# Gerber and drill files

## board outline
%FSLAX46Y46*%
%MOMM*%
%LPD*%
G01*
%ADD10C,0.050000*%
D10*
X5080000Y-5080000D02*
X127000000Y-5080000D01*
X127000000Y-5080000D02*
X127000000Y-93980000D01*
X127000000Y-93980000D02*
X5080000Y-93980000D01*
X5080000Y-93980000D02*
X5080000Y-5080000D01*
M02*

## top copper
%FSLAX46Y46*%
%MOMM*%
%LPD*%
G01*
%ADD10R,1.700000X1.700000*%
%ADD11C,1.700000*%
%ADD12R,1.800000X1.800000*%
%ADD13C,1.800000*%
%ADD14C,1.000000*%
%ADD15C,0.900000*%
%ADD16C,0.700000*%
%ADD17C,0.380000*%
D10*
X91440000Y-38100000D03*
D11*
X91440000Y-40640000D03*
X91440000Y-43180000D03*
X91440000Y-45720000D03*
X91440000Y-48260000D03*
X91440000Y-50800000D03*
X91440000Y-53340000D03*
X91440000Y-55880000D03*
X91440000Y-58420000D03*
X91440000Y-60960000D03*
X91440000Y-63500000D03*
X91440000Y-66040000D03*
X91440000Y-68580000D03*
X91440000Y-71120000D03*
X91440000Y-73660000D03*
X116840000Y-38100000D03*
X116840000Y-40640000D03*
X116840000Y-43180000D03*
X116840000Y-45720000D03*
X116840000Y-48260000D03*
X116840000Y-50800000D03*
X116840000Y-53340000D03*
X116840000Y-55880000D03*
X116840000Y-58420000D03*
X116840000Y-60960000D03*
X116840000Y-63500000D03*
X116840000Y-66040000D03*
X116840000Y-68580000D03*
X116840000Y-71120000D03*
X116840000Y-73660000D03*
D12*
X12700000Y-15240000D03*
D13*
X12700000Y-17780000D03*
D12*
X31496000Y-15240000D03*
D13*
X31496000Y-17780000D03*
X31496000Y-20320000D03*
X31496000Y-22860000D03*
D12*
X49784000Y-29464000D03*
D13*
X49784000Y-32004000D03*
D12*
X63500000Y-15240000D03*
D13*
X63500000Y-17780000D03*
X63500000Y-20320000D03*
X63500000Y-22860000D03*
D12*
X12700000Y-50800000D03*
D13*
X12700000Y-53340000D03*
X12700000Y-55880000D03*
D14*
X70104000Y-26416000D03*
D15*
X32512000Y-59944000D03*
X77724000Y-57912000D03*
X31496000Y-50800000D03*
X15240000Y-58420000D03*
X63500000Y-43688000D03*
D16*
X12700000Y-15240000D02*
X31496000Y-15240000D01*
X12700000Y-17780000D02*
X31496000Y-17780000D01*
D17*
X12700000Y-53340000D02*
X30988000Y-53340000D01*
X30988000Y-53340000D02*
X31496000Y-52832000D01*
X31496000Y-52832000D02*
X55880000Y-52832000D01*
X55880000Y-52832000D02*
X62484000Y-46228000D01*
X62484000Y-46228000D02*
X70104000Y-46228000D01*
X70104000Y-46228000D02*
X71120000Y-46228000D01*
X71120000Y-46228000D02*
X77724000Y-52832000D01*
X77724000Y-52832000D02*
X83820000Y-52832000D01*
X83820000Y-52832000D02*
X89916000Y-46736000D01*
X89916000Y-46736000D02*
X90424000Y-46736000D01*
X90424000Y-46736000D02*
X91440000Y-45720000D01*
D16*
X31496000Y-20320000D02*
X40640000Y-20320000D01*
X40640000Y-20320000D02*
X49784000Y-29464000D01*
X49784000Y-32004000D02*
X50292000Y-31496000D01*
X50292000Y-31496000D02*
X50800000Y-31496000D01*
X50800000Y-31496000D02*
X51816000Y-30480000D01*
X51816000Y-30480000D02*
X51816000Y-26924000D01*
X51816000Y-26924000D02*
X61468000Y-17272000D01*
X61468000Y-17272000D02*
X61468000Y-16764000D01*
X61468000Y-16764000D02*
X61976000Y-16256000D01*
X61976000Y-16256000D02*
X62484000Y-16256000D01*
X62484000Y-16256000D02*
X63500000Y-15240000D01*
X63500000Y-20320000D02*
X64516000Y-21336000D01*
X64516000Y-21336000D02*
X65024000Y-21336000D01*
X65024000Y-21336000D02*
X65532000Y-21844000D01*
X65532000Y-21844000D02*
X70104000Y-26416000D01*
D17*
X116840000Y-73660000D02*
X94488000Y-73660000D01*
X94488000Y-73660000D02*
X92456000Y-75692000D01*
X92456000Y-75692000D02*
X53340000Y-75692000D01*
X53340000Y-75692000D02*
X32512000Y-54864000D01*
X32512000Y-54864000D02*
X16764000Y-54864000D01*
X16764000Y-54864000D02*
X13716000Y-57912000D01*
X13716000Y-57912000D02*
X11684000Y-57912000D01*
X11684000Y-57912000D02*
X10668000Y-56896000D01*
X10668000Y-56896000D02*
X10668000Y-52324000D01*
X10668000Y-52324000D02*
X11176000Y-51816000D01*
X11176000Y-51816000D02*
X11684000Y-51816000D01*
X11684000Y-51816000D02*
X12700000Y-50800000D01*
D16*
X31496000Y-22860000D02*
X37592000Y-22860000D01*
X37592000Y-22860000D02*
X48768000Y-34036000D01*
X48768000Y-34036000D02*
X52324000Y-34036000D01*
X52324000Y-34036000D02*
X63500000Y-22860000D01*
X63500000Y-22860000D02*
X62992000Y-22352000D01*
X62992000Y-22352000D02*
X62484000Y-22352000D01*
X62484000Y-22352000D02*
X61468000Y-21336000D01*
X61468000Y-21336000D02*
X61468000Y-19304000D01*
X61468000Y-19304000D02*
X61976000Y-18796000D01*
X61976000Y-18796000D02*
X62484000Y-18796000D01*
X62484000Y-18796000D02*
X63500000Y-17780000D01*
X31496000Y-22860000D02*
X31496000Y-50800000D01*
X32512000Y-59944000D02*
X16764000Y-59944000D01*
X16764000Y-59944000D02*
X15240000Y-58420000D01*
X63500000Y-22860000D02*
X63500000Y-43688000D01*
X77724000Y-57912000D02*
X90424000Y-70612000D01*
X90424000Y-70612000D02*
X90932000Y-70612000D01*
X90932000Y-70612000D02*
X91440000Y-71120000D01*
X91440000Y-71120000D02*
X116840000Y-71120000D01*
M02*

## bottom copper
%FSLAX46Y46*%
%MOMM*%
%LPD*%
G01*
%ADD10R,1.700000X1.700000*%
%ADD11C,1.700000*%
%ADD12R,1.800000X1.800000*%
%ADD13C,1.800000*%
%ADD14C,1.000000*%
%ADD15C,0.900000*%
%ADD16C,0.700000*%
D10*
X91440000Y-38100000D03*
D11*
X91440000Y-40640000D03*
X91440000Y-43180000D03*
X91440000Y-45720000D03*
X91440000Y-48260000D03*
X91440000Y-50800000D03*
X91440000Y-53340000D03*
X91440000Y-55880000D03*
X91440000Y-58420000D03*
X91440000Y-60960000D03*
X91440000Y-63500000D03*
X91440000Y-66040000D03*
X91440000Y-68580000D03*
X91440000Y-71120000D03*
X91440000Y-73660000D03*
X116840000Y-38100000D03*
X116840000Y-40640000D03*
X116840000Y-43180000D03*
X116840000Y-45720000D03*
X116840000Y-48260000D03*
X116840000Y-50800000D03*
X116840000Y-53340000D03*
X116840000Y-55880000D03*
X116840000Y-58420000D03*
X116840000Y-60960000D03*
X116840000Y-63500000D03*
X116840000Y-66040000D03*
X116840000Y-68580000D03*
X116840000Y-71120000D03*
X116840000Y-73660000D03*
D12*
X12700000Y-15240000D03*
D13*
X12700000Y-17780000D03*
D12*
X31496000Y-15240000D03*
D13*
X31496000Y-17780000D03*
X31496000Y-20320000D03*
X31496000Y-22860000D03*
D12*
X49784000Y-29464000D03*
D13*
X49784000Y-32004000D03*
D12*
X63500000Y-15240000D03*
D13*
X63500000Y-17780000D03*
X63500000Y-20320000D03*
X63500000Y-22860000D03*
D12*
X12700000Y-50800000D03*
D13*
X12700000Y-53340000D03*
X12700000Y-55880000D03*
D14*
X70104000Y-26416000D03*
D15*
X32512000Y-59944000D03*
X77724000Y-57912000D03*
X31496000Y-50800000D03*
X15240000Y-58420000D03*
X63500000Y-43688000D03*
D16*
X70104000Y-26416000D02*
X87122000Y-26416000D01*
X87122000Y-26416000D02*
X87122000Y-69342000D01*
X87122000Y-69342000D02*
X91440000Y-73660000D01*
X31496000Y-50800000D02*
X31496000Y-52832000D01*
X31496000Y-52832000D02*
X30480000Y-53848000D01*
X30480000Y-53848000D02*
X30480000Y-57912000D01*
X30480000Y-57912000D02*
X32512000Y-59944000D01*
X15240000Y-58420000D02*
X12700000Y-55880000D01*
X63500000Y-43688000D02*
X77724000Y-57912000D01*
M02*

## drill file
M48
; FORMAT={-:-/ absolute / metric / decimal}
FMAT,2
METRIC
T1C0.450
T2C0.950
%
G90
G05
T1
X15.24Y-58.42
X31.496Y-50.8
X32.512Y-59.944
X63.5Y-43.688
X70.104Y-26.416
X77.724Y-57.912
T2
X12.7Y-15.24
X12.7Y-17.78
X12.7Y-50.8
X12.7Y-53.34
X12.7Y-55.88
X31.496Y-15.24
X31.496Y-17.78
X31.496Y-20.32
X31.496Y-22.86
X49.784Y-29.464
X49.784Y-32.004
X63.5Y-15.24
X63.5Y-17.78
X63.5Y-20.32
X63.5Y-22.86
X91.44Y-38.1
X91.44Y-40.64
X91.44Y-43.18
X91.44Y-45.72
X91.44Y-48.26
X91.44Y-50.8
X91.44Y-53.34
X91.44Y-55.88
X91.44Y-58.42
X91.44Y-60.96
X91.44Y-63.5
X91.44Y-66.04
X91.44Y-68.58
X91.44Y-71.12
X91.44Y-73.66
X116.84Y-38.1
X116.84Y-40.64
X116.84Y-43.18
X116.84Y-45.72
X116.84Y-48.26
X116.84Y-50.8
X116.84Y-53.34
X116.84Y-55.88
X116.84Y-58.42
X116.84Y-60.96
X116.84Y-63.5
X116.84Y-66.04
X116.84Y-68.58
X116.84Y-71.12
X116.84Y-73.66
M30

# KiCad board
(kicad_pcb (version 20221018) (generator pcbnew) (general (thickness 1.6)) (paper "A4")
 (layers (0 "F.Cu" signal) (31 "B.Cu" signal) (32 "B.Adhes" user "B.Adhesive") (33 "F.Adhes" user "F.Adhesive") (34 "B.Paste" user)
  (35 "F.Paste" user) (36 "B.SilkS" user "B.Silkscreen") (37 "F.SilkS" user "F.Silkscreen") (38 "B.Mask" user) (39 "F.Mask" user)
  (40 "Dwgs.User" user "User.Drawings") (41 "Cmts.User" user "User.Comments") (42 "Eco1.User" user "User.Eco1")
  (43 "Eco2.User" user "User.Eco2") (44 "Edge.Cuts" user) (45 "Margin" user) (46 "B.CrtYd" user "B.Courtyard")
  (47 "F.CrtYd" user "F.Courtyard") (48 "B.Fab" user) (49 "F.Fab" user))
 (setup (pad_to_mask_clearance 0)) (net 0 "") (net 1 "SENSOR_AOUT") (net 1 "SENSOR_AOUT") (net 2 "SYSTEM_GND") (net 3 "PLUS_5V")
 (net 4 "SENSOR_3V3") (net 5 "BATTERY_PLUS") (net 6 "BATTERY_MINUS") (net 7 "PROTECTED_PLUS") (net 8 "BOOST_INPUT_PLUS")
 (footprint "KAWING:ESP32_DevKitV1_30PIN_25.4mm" (layer "F.Cu") (at 91.44 38.1)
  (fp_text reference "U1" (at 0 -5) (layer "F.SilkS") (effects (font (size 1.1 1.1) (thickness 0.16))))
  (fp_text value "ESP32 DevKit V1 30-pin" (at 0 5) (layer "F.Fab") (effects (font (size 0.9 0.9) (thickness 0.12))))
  (pad "1" thru_hole rect (at 0 0) (size 1.7 1.7) (drill 0.95) (layers "*.Cu" "*.Mask"))
  (pad "2" thru_hole circle (at 0 2.54) (size 1.7 1.7) (drill 0.95) (layers "*.Cu" "*.Mask"))
  (pad "3" thru_hole circle (at 0 5.08) (size 1.7 1.7) (drill 0.95) (layers "*.Cu" "*.Mask"))
  (pad "4" thru_hole circle (at 0 7.62) (size 1.7 1.7) (drill 0.95) (layers "*.Cu" "*.Mask") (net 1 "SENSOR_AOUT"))
  (pad "5" thru_hole circle (at 0 10.16) (size 1.7 1.7) (drill 0.95) (layers "*.Cu" "*.Mask"))
  (pad "6" thru_hole circle (at 0 12.7) (size 1.7 1.7) (drill 0.95) (layers "*.Cu" "*.Mask"))
  (pad "7" thru_hole circle (at 0 15.24) (size 1.7 1.7) (drill 0.95) (layers "*.Cu" "*.Mask"))
  (pad "8" thru_hole circle (at 0 17.78) (size 1.7 1.7) (drill 0.95) (layers "*.Cu" "*.Mask"))
  (pad "9" thru_hole circle (at 0 20.32) (size 1.7 1.7) (drill 0.95) (layers "*.Cu" "*.Mask"))
  (pad "10" thru_hole circle (at 0 22.86) (size 1.7 1.7) (drill 0.95) (layers "*.Cu" "*.Mask"))
  (pad "11" thru_hole circle (at 0 25.4) (size 1.7 1.7) (drill 0.95) (layers "*.Cu" "*.Mask"))
  (pad "12" thru_hole circle (at 0 27.94) (size 1.7 1.7) (drill 0.95) (layers "*.Cu" "*.Mask"))
  (pad "13" thru_hole circle (at 0 30.48) (size 1.7 1.7) (drill 0.95) (layers "*.Cu" "*.Mask"))
  (pad "14" thru_hole circle (at 0 33.02) (size 1.7 1.7) (drill 0.95) (layers "*.Cu" "*.Mask") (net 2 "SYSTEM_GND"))
  (pad "15" thru_hole circle (at 0 35.56) (size 1.7 1.7) (drill 0.95) (layers "*.Cu" "*.Mask") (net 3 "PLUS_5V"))
  (pad "16" thru_hole circle (at 25.4 0) (size 1.7 1.7) (drill 0.95) (layers "*.Cu" "*.Mask"))
  (pad "17" thru_hole circle (at 25.4 2.54) (size 1.7 1.7) (drill 0.95) (layers "*.Cu" "*.Mask"))
  (pad "18" thru_hole circle (at 25.4 5.08) (size 1.7 1.7) (drill 0.95) (layers "*.Cu" "*.Mask"))
  (pad "19" thru_hole circle (at 25.4 7.62) (size 1.7 1.7) (drill 0.95) (layers "*.Cu" "*.Mask"))
  (pad "20" thru_hole circle (at 25.4 10.16) (size 1.7 1.7) (drill 0.95) (layers "*.Cu" "*.Mask"))
  (pad "21" thru_hole circle (at 25.4 12.7) (size 1.7 1.7) (drill 0.95) (layers "*.Cu" "*.Mask"))
  (pad "22" thru_hole circle (at 25.4 15.24) (size 1.7 1.7) (drill 0.95) (layers "*.Cu" "*.Mask"))
  (pad "23" thru_hole circle (at 25.4 17.78) (size 1.7 1.7) (drill 0.95) (layers "*.Cu" "*.Mask"))
  (pad "24" thru_hole circle (at 25.4 20.32) (size 1.7 1.7) (drill 0.95) (layers "*.Cu" "*.Mask"))
  (pad "25" thru_hole circle (at 25.4 22.86) (size 1.7 1.7) (drill 0.95) (layers "*.Cu" "*.Mask"))
  (pad "26" thru_hole circle (at 25.4 25.4) (size 1.7 1.7) (drill 0.95) (layers "*.Cu" "*.Mask"))
  (pad "27" thru_hole circle (at 25.4 27.94) (size 1.7 1.7) (drill 0.95) (layers "*.Cu" "*.Mask"))
  (pad "28" thru_hole circle (at 25.4 30.48) (size 1.7 1.7) (drill 0.95) (layers "*.Cu" "*.Mask"))
  (pad "29" thru_hole circle (at 25.4 33.02) (size 1.7 1.7) (drill 0.95) (layers "*.Cu" "*.Mask") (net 2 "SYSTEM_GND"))
  (pad "30" thru_hole circle (at 25.4 35.56) (size 1.7 1.7) (drill 0.95) (layers "*.Cu" "*.Mask") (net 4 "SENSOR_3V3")))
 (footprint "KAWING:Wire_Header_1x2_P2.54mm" (layer "F.Cu") (at 12.7 15.24)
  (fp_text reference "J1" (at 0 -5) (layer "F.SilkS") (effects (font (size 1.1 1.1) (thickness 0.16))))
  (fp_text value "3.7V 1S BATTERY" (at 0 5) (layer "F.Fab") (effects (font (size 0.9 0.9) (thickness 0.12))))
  (pad "1" thru_hole rect (at 0 0) (size 1.8 1.8) (drill 0.95) (layers "*.Cu" "*.Mask") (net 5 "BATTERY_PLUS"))
  (pad "2" thru_hole circle (at 0 2.54) (size 1.8 1.8) (drill 0.95) (layers "*.Cu" "*.Mask") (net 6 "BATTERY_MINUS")))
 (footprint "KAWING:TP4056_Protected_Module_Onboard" (layer "F.Cu") (at 31.496 15.24)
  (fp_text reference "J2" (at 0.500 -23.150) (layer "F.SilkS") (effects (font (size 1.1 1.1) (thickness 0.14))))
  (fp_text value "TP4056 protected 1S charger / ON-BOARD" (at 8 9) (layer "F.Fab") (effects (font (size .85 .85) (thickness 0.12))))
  (pad "1" thru_hole rect (at 0.0 0.0) (size 1.8 1.8) (drill 0.95) (layers "*.Cu" "*.Mask") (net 5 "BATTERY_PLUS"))
  (pad "2" thru_hole circle (at 0.0 2.54) (size 1.8 1.8) (drill 0.95) (layers "*.Cu" "*.Mask") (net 6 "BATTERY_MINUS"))
  (pad "3" thru_hole circle (at 0.0 5.08) (size 1.8 1.8) (drill 0.95) (layers "*.Cu" "*.Mask") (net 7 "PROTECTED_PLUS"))
  (pad "4" thru_hole circle (at 0.0 7.62) (size 1.8 1.8) (drill 0.95) (layers "*.Cu" "*.Mask") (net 2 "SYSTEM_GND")))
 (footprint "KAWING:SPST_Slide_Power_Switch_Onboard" (layer "F.Cu") (at 49.784 29.464)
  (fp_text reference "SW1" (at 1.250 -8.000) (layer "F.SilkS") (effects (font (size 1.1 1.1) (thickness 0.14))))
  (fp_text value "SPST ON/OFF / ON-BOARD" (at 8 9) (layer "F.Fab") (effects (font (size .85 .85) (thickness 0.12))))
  (pad "1" thru_hole rect (at 0.0 0.0) (size 1.8 1.8) (drill 0.95) (layers "*.Cu" "*.Mask") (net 7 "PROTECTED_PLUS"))
  (pad "2" thru_hole circle (at 0.0 2.54) (size 1.8 1.8) (drill 0.95) (layers "*.Cu" "*.Mask") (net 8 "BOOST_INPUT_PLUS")))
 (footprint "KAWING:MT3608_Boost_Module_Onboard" (layer "F.Cu") (at 63.5 15.24)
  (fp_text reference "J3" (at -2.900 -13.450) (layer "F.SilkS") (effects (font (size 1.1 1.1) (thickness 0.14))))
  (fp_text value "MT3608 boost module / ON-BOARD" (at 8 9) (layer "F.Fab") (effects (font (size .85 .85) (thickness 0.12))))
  (pad "1" thru_hole rect (at 0.0 0.0) (size 1.8 1.8) (drill 0.95) (layers "*.Cu" "*.Mask") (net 8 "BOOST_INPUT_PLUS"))
  (pad "2" thru_hole circle (at 0.0 2.54) (size 1.8 1.8) (drill 0.95) (layers "*.Cu" "*.Mask") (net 2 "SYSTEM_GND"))
  (pad "3" thru_hole circle (at 0.0 5.08) (size 1.8 1.8) (drill 0.95) (layers "*.Cu" "*.Mask") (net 3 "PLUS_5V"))
  (pad "4" thru_hole circle (at 0.0 7.62) (size 1.8 1.8) (drill 0.95) (layers "*.Cu" "*.Mask") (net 2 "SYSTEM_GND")))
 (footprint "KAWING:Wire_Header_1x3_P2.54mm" (layer "F.Cu") (at 12.7 50.8)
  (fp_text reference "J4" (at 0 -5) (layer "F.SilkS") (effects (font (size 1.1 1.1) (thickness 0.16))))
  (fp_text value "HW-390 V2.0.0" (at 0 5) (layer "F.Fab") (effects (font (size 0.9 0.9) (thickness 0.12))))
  (pad "1" thru_hole rect (at 0 0) (size 1.8 1.8) (drill 0.95) (layers "*.Cu" "*.Mask") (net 4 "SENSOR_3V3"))
  (pad "2" thru_hole circle (at 0 2.54) (size 1.8 1.8) (drill 0.95) (layers "*.Cu" "*.Mask") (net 1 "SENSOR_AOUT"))
  (pad "3" thru_hole circle (at 0 5.08) (size 1.8 1.8) (drill 0.95) (layers "*.Cu" "*.Mask") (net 2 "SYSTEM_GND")))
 (gr_line (start 5.08 5.08) (end 127 5.08) (stroke (width 0.05) (type default)) (layer "Edge.Cuts"))
 (gr_line (start 127 5.08) (end 127 93.98) (stroke (width 0.05) (type default)) (layer "Edge.Cuts"))
 (gr_line (start 127 93.98) (end 5.08 93.98) (stroke (width 0.05) (type default)) (layer "Edge.Cuts"))
 (gr_line (start 5.08 93.98) (end 5.08 5.08) (stroke (width 0.05) (type default)) (layer "Edge.Cuts"))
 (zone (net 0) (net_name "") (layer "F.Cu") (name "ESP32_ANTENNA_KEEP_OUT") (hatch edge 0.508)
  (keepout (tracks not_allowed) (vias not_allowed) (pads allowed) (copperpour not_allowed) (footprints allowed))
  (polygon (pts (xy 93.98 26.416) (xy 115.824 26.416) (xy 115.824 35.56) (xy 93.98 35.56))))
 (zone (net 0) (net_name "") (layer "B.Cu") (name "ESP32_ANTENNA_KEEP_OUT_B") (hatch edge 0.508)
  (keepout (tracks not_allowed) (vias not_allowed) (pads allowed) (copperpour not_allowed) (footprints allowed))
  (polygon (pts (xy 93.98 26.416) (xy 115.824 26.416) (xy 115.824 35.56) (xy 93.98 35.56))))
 (segment (start 12.7 15.24) (end 31.496 15.24) (width 0.7) (layer "F.Cu") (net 5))
 (segment (start 12.7 17.78) (end 31.496 17.78) (width 0.7) (layer "F.Cu") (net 6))
 (segment (start 12.7 53.34) (end 30.988 53.34) (width 0.38) (layer "F.Cu") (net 1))
 (segment (start 30.988 53.34) (end 31.496 52.832) (width 0.38) (layer "F.Cu") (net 1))
 (segment (start 31.496 52.832) (end 55.88 52.832) (width 0.38) (layer "F.Cu") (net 1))
 (segment (start 55.88 52.832) (end 62.484 46.228) (width 0.38) (layer "F.Cu") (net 1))
 (segment (start 62.484 46.228) (end 70.104 46.228) (width 0.38) (layer "F.Cu") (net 1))
 (segment (start 70.104 46.228) (end 71.12 46.228) (width 0.38) (layer "F.Cu") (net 1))
 (segment (start 71.12 46.228) (end 77.724 52.832) (width 0.38) (layer "F.Cu") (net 1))
 (segment (start 77.724 52.832) (end 83.82 52.832) (width 0.38) (layer "F.Cu") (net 1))
 (segment (start 83.82 52.832) (end 89.916 46.736) (width 0.38) (layer "F.Cu") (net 1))
 (segment (start 89.916 46.736) (end 90.424 46.736) (width 0.38) (layer "F.Cu") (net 1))
 (segment (start 90.424 46.736) (end 91.44 45.72) (width 0.38) (layer "F.Cu") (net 1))
 (segment (start 31.496 20.32) (end 40.64 20.32) (width 0.7) (layer "F.Cu") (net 7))
 (segment (start 40.64 20.32) (end 49.784 29.464) (width 0.7) (layer "F.Cu") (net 7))
 (segment (start 49.784 32.004) (end 50.292 31.496) (width 0.7) (layer "F.Cu") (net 8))
 (segment (start 50.292 31.496) (end 50.8 31.496) (width 0.7) (layer "F.Cu") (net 8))
 (segment (start 50.8 31.496) (end 51.816 30.48) (width 0.7) (layer "F.Cu") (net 8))
 (segment (start 51.816 30.48) (end 51.816 26.924) (width 0.7) (layer "F.Cu") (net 8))
 (segment (start 51.816 26.924) (end 61.468 17.272) (width 0.7) (layer "F.Cu") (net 8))
 (segment (start 61.468 17.272) (end 61.468 16.764) (width 0.7) (layer "F.Cu") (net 8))
 (segment (start 61.468 16.764) (end 61.976 16.256) (width 0.7) (layer "F.Cu") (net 8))
 (segment (start 61.976 16.256) (end 62.484 16.256) (width 0.7) (layer "F.Cu") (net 8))
 (segment (start 62.484 16.256) (end 63.5 15.24) (width 0.7) (layer "F.Cu") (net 8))
 (segment (start 63.5 20.32) (end 64.516 21.336) (width 0.7) (layer "F.Cu") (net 3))
 (segment (start 64.516 21.336) (end 65.024 21.336) (width 0.7) (layer "F.Cu") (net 3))
 (segment (start 65.024 21.336) (end 65.532 21.844) (width 0.7) (layer "F.Cu") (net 3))
 (segment (start 65.532 21.844) (end 70.104 26.416) (width 0.7) (layer "F.Cu") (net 3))
 (segment (start 70.104 26.416) (end 87.122 26.416) (width 0.7) (layer "B.Cu") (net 3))
 (segment (start 87.122 26.416) (end 87.122 69.342) (width 0.7) (layer "B.Cu") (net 3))
 (segment (start 87.122 69.342) (end 91.44 73.66) (width 0.7) (layer "B.Cu") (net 3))
 (via (at 70.104 26.416) (size 1.0) (drill 0.45) (layers "F.Cu" "B.Cu") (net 3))
 (segment (start 116.84 73.66) (end 94.488 73.66) (width 0.38) (layer "F.Cu") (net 4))
 (segment (start 94.488 73.66) (end 92.456 75.692) (width 0.38) (layer "F.Cu") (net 4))
 (segment (start 92.456 75.692) (end 53.34 75.692) (width 0.38) (layer "F.Cu") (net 4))
 (segment (start 53.34 75.692) (end 32.512 54.864) (width 0.38) (layer "F.Cu") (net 4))
 (segment (start 32.512 54.864) (end 16.764 54.864) (width 0.38) (layer "F.Cu") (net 4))
 (segment (start 16.764 54.864) (end 13.716 57.912) (width 0.38) (layer "F.Cu") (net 4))
 (segment (start 13.716 57.912) (end 11.684 57.912) (width 0.38) (layer "F.Cu") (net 4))
 (segment (start 11.684 57.912) (end 10.668 56.896) (width 0.38) (layer "F.Cu") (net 4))
 (segment (start 10.668 56.896) (end 10.668 52.324) (width 0.38) (layer "F.Cu") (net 4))
 (segment (start 10.668 52.324) (end 11.176 51.816) (width 0.38) (layer "F.Cu") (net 4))
 (segment (start 11.176 51.816) (end 11.684 51.816) (width 0.38) (layer "F.Cu") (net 4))
 (segment (start 11.684 51.816) (end 12.7 50.8) (width 0.38) (layer "F.Cu") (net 4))
 (via (at 32.512 59.944) (size 0.9) (drill 0.45) (layers "F.Cu" "B.Cu") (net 2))
 (via (at 77.724 57.912) (size 0.9) (drill 0.45) (layers "F.Cu" "B.Cu") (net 2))
 (segment (start 31.496 22.86) (end 37.592 22.86) (width 0.7) (layer "F.Cu") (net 2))
 (segment (start 37.592 22.86) (end 48.768 34.036) (width 0.7) (layer "F.Cu") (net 2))
 (segment (start 48.768 34.036) (end 52.324 34.036) (width 0.7) (layer "F.Cu") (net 2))
 (segment (start 52.324 34.036) (end 63.5 22.86) (width 0.7) (layer "F.Cu") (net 2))
 (segment (start 63.5 22.86) (end 62.992 22.352) (width 0.7) (layer "F.Cu") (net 2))
 (segment (start 62.992 22.352) (end 62.484 22.352) (width 0.7) (layer "F.Cu") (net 2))
 (segment (start 62.484 22.352) (end 61.468 21.336) (width 0.7) (layer "F.Cu") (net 2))
 (segment (start 61.468 21.336) (end 61.468 19.304) (width 0.7) (layer "F.Cu") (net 2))
 (segment (start 61.468 19.304) (end 61.976 18.796) (width 0.7) (layer "F.Cu") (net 2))
 (segment (start 61.976 18.796) (end 62.484 18.796) (width 0.7) (layer "F.Cu") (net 2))
 (segment (start 62.484 18.796) (end 63.5 17.78) (width 0.7) (layer "F.Cu") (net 2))
 (segment (start 31.496 22.86) (end 31.496 50.8) (width 0.7) (layer "F.Cu") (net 2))
 (segment (start 31.496 50.8) (end 31.496 52.832) (width 0.7) (layer "B.Cu") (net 2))
 (segment (start 31.496 52.832) (end 30.48 53.848) (width 0.7) (layer "B.Cu") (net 2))
 (segment (start 30.48 53.848) (end 30.48 57.912) (width 0.7) (layer "B.Cu") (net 2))
 (segment (start 30.48 57.912) (end 32.512 59.944) (width 0.7) (layer "B.Cu") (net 2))
 (via (at 31.496 50.8) (size 0.9) (drill 0.45) (layers "F.Cu" "B.Cu") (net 2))
 (segment (start 32.512 59.944) (end 16.764 59.944) (width 0.7) (layer "F.Cu") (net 2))
 (segment (start 16.764 59.944) (end 15.24 58.42) (width 0.7) (layer "F.Cu") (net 2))
 (segment (start 15.24 58.42) (end 12.7 55.88) (width 0.7) (layer "B.Cu") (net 2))
 (via (at 15.24 58.42) (size 0.9) (drill 0.45) (layers "F.Cu" "B.Cu") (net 2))
 (segment (start 63.5 22.86) (end 63.5 43.688) (width 0.7) (layer "F.Cu") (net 2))
 (segment (start 63.5 43.688) (end 77.724 57.912) (width 0.7) (layer "B.Cu") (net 2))
 (via (at 63.5 43.688) (size 0.9) (drill 0.45) (layers "F.Cu" "B.Cu") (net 2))
 (segment (start 77.724 57.912) (end 90.424 70.612) (width 0.7) (layer "F.Cu") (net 2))
 (segment (start 90.424 70.612) (end 90.932 70.612) (width 0.7) (layer "F.Cu") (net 2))
 (segment (start 90.932 70.612) (end 91.44 71.12) (width 0.7) (layer "F.Cu") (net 2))
 (segment (start 91.44 71.12) (end 116.84 71.12) (width 0.7) (layer "F.Cu") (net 2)))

